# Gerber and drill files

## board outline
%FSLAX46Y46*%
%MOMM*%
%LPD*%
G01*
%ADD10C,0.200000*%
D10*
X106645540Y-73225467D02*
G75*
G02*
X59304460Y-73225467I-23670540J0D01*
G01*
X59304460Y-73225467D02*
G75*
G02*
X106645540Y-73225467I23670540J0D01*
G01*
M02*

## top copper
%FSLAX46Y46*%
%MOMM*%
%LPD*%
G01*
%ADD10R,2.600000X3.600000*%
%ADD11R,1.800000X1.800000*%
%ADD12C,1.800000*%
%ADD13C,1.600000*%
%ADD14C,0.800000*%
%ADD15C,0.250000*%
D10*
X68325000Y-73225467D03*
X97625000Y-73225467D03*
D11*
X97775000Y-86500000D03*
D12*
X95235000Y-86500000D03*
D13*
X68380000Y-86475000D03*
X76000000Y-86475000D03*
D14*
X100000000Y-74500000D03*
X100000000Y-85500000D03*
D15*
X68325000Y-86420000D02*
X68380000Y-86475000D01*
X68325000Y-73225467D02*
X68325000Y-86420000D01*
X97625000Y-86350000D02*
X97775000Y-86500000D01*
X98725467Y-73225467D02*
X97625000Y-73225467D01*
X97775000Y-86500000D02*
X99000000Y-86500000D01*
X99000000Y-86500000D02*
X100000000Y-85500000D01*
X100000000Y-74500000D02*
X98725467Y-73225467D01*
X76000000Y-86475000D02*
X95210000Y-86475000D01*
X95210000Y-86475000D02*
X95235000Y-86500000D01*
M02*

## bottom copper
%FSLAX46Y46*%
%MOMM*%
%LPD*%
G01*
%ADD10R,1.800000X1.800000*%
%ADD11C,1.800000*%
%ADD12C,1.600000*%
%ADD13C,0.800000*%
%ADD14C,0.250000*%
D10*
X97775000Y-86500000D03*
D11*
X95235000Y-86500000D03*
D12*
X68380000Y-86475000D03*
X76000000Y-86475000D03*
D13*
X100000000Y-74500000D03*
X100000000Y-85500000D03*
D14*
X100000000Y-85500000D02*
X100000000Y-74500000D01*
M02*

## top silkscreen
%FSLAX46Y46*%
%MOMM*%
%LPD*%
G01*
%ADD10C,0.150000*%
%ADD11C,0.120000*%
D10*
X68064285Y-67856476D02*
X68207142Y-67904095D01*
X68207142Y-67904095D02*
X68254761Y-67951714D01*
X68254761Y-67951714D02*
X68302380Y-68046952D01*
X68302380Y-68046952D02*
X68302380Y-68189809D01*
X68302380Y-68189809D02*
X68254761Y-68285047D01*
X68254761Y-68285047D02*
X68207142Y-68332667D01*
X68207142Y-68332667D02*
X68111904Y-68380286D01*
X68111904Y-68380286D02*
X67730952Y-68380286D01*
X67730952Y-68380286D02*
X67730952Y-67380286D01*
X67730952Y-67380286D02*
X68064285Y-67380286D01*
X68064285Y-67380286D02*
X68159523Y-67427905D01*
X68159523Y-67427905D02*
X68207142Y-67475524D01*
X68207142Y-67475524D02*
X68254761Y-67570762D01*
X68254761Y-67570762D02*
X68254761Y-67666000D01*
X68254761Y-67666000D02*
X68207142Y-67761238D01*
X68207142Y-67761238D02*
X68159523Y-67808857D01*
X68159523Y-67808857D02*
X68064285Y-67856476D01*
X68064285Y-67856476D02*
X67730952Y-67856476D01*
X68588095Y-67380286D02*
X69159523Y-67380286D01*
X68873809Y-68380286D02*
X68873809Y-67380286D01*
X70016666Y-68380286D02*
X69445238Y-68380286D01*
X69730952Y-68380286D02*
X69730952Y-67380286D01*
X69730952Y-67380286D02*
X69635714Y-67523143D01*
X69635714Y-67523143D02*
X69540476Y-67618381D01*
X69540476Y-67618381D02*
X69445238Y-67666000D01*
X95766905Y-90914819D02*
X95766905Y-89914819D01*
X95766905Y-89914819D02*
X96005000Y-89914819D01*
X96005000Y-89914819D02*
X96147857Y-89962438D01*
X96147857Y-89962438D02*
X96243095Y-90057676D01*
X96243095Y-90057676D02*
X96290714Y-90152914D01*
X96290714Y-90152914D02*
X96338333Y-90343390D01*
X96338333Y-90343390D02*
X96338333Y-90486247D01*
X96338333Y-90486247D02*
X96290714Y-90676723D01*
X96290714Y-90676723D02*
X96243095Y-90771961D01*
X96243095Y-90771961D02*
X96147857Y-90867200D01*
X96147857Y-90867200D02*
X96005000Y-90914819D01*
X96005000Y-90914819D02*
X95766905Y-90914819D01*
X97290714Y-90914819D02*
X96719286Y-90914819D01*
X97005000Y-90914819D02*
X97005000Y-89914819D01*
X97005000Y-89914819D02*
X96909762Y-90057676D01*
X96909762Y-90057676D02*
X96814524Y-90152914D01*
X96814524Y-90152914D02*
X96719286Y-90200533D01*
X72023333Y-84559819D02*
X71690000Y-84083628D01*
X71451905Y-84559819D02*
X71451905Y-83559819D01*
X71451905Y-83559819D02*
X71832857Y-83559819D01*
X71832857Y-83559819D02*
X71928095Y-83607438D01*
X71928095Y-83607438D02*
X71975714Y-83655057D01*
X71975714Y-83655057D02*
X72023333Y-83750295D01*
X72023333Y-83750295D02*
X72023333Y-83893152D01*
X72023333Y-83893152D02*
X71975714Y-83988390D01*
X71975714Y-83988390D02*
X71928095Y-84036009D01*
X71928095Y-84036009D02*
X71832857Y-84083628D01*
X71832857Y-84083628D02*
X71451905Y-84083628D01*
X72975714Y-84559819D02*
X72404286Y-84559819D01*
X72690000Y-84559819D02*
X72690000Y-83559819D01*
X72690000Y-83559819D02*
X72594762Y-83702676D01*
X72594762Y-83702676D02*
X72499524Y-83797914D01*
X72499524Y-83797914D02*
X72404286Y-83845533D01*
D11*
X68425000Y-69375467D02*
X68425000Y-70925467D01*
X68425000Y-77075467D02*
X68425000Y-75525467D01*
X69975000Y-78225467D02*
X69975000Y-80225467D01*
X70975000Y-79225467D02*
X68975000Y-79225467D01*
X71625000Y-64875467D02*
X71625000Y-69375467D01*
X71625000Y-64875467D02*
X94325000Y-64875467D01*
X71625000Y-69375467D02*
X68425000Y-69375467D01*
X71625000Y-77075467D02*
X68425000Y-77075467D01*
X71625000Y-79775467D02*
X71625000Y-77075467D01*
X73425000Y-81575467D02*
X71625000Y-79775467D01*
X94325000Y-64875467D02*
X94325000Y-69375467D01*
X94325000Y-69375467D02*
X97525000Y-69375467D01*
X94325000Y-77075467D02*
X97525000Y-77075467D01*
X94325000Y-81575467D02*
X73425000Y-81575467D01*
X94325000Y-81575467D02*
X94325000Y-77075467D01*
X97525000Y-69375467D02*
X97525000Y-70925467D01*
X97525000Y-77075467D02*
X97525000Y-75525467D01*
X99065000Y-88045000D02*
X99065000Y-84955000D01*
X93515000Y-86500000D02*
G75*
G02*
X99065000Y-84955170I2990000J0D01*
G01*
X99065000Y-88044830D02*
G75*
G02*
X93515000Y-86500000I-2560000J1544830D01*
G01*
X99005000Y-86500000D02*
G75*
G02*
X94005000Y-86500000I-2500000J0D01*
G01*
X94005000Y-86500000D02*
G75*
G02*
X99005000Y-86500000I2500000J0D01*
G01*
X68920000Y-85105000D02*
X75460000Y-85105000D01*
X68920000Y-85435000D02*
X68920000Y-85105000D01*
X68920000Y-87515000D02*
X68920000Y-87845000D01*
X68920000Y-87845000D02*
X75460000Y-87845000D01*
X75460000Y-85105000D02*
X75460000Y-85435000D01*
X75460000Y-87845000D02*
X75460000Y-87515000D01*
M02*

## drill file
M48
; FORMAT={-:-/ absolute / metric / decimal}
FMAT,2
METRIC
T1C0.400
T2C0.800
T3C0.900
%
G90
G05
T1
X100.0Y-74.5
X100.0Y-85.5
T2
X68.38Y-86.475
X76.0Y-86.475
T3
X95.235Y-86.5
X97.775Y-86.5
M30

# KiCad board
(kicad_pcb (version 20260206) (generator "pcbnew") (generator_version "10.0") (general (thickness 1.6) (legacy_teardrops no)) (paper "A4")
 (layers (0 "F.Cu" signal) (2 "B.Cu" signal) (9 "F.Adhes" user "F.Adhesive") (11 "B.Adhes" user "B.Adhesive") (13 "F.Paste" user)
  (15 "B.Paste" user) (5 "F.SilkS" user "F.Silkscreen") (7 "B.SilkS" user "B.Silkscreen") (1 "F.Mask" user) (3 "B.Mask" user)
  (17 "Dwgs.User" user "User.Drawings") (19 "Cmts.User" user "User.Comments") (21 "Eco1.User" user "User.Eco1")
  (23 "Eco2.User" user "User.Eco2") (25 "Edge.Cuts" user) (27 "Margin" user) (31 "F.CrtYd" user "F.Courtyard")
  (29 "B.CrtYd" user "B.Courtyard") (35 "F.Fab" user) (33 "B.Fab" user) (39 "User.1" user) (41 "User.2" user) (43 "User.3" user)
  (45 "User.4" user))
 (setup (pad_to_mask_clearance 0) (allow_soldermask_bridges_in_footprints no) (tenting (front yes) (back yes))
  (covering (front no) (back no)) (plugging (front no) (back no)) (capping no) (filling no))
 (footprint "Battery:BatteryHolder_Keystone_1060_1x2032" (layer "F.Cu") (at 82.975 73.225467)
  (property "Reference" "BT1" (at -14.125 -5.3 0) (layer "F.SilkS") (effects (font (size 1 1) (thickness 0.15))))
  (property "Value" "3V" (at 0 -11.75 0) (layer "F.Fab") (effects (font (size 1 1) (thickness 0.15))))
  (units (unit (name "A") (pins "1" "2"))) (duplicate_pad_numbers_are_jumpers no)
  (fp_line (start -14.55 -3.85) (end -14.55 -2.3) (stroke (width 0.12) (type solid)) (layer "F.SilkS"))
  (fp_line (start -14.55 3.85) (end -14.55 2.3) (stroke (width 0.12) (type solid)) (layer "F.SilkS"))
  (fp_line (start -13 5) (end -13 7) (stroke (width 0.12) (type solid)) (layer "F.SilkS"))
  (fp_line (start -12 6) (end -14 6) (stroke (width 0.12) (type solid)) (layer "F.SilkS"))
  (fp_line (start -11.35 -8.35) (end -11.35 -3.85) (stroke (width 0.12) (type solid)) (layer "F.SilkS"))
  (fp_line (start -11.35 -8.35) (end 11.35 -8.35) (stroke (width 0.12) (type solid)) (layer "F.SilkS"))
  (fp_line (start -11.35 -3.85) (end -14.55 -3.85) (stroke (width 0.12) (type solid)) (layer "F.SilkS"))
  (fp_line (start -11.35 3.85) (end -14.55 3.85) (stroke (width 0.12) (type solid)) (layer "F.SilkS"))
  (fp_line (start -11.35 6.55) (end -11.35 3.85) (stroke (width 0.12) (type solid)) (layer "F.SilkS"))
  (fp_line (start -9.55 8.35) (end -11.35 6.55) (stroke (width 0.12) (type solid)) (layer "F.SilkS"))
  (fp_line (start 11.35 -8.35) (end 11.35 -3.85) (stroke (width 0.12) (type solid)) (layer "F.SilkS"))
  (fp_line (start 11.35 -3.85) (end 14.55 -3.85) (stroke (width 0.12) (type solid)) (layer "F.SilkS"))
  (fp_line (start 11.35 3.85) (end 14.55 3.85) (stroke (width 0.12) (type solid)) (layer "F.SilkS"))
  (fp_line (start 11.35 8.35) (end -9.55 8.35) (stroke (width 0.12) (type solid)) (layer "F.SilkS"))
  (fp_line (start 11.35 8.35) (end 11.35 3.85) (stroke (width 0.12) (type solid)) (layer "F.SilkS"))
  (fp_line (start 14.55 -3.85) (end 14.55 -2.3) (stroke (width 0.12) (type solid)) (layer "F.SilkS"))
  (fp_line (start 14.55 3.85) (end 14.55 2.3) (stroke (width 0.12) (type solid)) (layer "F.SilkS"))
  (pad "1" smd rect (at -14.65 0 180) (size 2.6 3.6) (layers "F.Cu" "F.Mask" "F.Paste") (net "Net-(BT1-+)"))
  (pad "2" smd rect (at 14.65 0 180) (size 2.6 3.6) (layers "F.Cu" "F.Mask" "F.Paste") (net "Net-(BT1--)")))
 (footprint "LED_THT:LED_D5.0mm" (layer "F.Cu") (at 97.775 86.5 180)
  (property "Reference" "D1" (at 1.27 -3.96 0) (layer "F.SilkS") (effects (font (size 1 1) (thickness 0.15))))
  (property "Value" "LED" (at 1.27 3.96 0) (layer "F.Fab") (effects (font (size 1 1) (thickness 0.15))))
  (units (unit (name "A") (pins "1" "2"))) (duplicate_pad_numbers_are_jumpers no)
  (fp_line (start -1.29 -1.545) (end -1.29 1.545) (stroke (width 0.12) (type solid)) (layer "F.SilkS"))
  (fp_arc (start 4.26 0) (mid 2.071779 2.880495) (end -1.29 1.54483) (stroke (width 0.12) (type solid)) (layer "F.SilkS"))
  (fp_arc (start -1.29 -1.54483) (mid 2.071779 -2.880495) (end 4.26 0) (stroke (width 0.12) (type solid)) (layer "F.SilkS"))
  (fp_circle (center 1.27 0) (end 3.77 0) (stroke (width 0.12) (type solid)) (fill no) (layer "F.SilkS"))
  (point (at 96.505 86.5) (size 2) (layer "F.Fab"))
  (pad "1" thru_hole rect (at 0 0 180) (size 1.8 1.8) (drill 0.9) (layers "*.Cu" "*.Mask") (remove_unused_layers no) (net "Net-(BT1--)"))
  (pad "2" thru_hole circle (at 2.54 0 180) (size 1.8 1.8) (drill 0.9) (layers "*.Cu" "*.Mask") (remove_unused_layers no) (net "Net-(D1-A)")))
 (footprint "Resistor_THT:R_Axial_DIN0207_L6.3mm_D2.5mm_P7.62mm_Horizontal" (layer "F.Cu") (at 68.38 86.475)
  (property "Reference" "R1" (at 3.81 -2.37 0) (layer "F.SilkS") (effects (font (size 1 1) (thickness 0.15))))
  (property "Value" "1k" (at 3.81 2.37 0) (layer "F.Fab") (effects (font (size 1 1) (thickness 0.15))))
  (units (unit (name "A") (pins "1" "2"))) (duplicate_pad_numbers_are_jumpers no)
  (fp_line (start 0.54 -1.37) (end 7.08 -1.37) (stroke (width 0.12) (type solid)) (layer "F.SilkS"))
  (fp_line (start 0.54 -1.04) (end 0.54 -1.37) (stroke (width 0.12) (type solid)) (layer "F.SilkS"))
  (fp_line (start 0.54 1.04) (end 0.54 1.37) (stroke (width 0.12) (type solid)) (layer "F.SilkS"))
  (fp_line (start 0.54 1.37) (end 7.08 1.37) (stroke (width 0.12) (type solid)) (layer "F.SilkS"))
  (fp_line (start 7.08 -1.37) (end 7.08 -1.04) (stroke (width 0.12) (type solid)) (layer "F.SilkS"))
  (fp_line (start 7.08 1.37) (end 7.08 1.04) (stroke (width 0.12) (type solid)) (layer "F.SilkS"))
  (pad "1" thru_hole circle (at 0 0) (size 1.6 1.6) (drill 0.8) (layers "*.Cu" "*.Mask") (remove_unused_layers no) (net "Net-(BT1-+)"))
  (pad "2" thru_hole circle (at 7.62 0) (size 1.6 1.6) (drill 0.8) (layers "*.Cu" "*.Mask") (remove_unused_layers no) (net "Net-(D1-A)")))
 (gr_circle (center 82.975 73.225467) (end 105.5 80.5) (stroke (width 0.2) (type solid)) (fill no) (layer "Edge.Cuts"))
 (segment (start 68.325 86.42) (end 68.38 86.475) (width 0.25) (layer "F.Cu") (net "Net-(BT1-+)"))
 (segment (start 68.325 73.225467) (end 68.325 86.42) (width 0.25) (layer "F.Cu") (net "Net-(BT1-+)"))
 (segment (start 97.625 86.35) (end 97.775 86.5) (width 0.25) (layer "F.Cu") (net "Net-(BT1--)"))
 (segment (start 98.725467 73.225467) (end 97.625 73.225467) (width 0.25) (layer "F.Cu") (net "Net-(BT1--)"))
 (segment (start 97.775 86.5) (end 99 86.5) (width 0.25) (layer "F.Cu") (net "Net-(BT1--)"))
 (segment (start 99 86.5) (end 100 85.5) (width 0.25) (layer "F.Cu") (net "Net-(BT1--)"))
 (segment (start 100 74.5) (end 98.725467 73.225467) (width 0.25) (layer "F.Cu") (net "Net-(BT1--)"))
 (via (at 100 74.5) (size 0.8) (drill 0.4) (layers "F.Cu" "B.Cu") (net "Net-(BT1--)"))
 (via (at 100 85.5) (size 0.8) (drill 0.4) (layers "F.Cu" "B.Cu") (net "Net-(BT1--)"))
 (segment (start 100 85.5) (end 100 74.5) (width 0.25) (layer "B.Cu") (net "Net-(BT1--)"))
 (segment (start 76 86.475) (end 95.21 86.475) (width 0.25) (layer "F.Cu") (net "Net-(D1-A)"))
 (segment (start 95.21 86.475) (end 95.235 86.5) (width 0.25) (layer "F.Cu") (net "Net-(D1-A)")))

